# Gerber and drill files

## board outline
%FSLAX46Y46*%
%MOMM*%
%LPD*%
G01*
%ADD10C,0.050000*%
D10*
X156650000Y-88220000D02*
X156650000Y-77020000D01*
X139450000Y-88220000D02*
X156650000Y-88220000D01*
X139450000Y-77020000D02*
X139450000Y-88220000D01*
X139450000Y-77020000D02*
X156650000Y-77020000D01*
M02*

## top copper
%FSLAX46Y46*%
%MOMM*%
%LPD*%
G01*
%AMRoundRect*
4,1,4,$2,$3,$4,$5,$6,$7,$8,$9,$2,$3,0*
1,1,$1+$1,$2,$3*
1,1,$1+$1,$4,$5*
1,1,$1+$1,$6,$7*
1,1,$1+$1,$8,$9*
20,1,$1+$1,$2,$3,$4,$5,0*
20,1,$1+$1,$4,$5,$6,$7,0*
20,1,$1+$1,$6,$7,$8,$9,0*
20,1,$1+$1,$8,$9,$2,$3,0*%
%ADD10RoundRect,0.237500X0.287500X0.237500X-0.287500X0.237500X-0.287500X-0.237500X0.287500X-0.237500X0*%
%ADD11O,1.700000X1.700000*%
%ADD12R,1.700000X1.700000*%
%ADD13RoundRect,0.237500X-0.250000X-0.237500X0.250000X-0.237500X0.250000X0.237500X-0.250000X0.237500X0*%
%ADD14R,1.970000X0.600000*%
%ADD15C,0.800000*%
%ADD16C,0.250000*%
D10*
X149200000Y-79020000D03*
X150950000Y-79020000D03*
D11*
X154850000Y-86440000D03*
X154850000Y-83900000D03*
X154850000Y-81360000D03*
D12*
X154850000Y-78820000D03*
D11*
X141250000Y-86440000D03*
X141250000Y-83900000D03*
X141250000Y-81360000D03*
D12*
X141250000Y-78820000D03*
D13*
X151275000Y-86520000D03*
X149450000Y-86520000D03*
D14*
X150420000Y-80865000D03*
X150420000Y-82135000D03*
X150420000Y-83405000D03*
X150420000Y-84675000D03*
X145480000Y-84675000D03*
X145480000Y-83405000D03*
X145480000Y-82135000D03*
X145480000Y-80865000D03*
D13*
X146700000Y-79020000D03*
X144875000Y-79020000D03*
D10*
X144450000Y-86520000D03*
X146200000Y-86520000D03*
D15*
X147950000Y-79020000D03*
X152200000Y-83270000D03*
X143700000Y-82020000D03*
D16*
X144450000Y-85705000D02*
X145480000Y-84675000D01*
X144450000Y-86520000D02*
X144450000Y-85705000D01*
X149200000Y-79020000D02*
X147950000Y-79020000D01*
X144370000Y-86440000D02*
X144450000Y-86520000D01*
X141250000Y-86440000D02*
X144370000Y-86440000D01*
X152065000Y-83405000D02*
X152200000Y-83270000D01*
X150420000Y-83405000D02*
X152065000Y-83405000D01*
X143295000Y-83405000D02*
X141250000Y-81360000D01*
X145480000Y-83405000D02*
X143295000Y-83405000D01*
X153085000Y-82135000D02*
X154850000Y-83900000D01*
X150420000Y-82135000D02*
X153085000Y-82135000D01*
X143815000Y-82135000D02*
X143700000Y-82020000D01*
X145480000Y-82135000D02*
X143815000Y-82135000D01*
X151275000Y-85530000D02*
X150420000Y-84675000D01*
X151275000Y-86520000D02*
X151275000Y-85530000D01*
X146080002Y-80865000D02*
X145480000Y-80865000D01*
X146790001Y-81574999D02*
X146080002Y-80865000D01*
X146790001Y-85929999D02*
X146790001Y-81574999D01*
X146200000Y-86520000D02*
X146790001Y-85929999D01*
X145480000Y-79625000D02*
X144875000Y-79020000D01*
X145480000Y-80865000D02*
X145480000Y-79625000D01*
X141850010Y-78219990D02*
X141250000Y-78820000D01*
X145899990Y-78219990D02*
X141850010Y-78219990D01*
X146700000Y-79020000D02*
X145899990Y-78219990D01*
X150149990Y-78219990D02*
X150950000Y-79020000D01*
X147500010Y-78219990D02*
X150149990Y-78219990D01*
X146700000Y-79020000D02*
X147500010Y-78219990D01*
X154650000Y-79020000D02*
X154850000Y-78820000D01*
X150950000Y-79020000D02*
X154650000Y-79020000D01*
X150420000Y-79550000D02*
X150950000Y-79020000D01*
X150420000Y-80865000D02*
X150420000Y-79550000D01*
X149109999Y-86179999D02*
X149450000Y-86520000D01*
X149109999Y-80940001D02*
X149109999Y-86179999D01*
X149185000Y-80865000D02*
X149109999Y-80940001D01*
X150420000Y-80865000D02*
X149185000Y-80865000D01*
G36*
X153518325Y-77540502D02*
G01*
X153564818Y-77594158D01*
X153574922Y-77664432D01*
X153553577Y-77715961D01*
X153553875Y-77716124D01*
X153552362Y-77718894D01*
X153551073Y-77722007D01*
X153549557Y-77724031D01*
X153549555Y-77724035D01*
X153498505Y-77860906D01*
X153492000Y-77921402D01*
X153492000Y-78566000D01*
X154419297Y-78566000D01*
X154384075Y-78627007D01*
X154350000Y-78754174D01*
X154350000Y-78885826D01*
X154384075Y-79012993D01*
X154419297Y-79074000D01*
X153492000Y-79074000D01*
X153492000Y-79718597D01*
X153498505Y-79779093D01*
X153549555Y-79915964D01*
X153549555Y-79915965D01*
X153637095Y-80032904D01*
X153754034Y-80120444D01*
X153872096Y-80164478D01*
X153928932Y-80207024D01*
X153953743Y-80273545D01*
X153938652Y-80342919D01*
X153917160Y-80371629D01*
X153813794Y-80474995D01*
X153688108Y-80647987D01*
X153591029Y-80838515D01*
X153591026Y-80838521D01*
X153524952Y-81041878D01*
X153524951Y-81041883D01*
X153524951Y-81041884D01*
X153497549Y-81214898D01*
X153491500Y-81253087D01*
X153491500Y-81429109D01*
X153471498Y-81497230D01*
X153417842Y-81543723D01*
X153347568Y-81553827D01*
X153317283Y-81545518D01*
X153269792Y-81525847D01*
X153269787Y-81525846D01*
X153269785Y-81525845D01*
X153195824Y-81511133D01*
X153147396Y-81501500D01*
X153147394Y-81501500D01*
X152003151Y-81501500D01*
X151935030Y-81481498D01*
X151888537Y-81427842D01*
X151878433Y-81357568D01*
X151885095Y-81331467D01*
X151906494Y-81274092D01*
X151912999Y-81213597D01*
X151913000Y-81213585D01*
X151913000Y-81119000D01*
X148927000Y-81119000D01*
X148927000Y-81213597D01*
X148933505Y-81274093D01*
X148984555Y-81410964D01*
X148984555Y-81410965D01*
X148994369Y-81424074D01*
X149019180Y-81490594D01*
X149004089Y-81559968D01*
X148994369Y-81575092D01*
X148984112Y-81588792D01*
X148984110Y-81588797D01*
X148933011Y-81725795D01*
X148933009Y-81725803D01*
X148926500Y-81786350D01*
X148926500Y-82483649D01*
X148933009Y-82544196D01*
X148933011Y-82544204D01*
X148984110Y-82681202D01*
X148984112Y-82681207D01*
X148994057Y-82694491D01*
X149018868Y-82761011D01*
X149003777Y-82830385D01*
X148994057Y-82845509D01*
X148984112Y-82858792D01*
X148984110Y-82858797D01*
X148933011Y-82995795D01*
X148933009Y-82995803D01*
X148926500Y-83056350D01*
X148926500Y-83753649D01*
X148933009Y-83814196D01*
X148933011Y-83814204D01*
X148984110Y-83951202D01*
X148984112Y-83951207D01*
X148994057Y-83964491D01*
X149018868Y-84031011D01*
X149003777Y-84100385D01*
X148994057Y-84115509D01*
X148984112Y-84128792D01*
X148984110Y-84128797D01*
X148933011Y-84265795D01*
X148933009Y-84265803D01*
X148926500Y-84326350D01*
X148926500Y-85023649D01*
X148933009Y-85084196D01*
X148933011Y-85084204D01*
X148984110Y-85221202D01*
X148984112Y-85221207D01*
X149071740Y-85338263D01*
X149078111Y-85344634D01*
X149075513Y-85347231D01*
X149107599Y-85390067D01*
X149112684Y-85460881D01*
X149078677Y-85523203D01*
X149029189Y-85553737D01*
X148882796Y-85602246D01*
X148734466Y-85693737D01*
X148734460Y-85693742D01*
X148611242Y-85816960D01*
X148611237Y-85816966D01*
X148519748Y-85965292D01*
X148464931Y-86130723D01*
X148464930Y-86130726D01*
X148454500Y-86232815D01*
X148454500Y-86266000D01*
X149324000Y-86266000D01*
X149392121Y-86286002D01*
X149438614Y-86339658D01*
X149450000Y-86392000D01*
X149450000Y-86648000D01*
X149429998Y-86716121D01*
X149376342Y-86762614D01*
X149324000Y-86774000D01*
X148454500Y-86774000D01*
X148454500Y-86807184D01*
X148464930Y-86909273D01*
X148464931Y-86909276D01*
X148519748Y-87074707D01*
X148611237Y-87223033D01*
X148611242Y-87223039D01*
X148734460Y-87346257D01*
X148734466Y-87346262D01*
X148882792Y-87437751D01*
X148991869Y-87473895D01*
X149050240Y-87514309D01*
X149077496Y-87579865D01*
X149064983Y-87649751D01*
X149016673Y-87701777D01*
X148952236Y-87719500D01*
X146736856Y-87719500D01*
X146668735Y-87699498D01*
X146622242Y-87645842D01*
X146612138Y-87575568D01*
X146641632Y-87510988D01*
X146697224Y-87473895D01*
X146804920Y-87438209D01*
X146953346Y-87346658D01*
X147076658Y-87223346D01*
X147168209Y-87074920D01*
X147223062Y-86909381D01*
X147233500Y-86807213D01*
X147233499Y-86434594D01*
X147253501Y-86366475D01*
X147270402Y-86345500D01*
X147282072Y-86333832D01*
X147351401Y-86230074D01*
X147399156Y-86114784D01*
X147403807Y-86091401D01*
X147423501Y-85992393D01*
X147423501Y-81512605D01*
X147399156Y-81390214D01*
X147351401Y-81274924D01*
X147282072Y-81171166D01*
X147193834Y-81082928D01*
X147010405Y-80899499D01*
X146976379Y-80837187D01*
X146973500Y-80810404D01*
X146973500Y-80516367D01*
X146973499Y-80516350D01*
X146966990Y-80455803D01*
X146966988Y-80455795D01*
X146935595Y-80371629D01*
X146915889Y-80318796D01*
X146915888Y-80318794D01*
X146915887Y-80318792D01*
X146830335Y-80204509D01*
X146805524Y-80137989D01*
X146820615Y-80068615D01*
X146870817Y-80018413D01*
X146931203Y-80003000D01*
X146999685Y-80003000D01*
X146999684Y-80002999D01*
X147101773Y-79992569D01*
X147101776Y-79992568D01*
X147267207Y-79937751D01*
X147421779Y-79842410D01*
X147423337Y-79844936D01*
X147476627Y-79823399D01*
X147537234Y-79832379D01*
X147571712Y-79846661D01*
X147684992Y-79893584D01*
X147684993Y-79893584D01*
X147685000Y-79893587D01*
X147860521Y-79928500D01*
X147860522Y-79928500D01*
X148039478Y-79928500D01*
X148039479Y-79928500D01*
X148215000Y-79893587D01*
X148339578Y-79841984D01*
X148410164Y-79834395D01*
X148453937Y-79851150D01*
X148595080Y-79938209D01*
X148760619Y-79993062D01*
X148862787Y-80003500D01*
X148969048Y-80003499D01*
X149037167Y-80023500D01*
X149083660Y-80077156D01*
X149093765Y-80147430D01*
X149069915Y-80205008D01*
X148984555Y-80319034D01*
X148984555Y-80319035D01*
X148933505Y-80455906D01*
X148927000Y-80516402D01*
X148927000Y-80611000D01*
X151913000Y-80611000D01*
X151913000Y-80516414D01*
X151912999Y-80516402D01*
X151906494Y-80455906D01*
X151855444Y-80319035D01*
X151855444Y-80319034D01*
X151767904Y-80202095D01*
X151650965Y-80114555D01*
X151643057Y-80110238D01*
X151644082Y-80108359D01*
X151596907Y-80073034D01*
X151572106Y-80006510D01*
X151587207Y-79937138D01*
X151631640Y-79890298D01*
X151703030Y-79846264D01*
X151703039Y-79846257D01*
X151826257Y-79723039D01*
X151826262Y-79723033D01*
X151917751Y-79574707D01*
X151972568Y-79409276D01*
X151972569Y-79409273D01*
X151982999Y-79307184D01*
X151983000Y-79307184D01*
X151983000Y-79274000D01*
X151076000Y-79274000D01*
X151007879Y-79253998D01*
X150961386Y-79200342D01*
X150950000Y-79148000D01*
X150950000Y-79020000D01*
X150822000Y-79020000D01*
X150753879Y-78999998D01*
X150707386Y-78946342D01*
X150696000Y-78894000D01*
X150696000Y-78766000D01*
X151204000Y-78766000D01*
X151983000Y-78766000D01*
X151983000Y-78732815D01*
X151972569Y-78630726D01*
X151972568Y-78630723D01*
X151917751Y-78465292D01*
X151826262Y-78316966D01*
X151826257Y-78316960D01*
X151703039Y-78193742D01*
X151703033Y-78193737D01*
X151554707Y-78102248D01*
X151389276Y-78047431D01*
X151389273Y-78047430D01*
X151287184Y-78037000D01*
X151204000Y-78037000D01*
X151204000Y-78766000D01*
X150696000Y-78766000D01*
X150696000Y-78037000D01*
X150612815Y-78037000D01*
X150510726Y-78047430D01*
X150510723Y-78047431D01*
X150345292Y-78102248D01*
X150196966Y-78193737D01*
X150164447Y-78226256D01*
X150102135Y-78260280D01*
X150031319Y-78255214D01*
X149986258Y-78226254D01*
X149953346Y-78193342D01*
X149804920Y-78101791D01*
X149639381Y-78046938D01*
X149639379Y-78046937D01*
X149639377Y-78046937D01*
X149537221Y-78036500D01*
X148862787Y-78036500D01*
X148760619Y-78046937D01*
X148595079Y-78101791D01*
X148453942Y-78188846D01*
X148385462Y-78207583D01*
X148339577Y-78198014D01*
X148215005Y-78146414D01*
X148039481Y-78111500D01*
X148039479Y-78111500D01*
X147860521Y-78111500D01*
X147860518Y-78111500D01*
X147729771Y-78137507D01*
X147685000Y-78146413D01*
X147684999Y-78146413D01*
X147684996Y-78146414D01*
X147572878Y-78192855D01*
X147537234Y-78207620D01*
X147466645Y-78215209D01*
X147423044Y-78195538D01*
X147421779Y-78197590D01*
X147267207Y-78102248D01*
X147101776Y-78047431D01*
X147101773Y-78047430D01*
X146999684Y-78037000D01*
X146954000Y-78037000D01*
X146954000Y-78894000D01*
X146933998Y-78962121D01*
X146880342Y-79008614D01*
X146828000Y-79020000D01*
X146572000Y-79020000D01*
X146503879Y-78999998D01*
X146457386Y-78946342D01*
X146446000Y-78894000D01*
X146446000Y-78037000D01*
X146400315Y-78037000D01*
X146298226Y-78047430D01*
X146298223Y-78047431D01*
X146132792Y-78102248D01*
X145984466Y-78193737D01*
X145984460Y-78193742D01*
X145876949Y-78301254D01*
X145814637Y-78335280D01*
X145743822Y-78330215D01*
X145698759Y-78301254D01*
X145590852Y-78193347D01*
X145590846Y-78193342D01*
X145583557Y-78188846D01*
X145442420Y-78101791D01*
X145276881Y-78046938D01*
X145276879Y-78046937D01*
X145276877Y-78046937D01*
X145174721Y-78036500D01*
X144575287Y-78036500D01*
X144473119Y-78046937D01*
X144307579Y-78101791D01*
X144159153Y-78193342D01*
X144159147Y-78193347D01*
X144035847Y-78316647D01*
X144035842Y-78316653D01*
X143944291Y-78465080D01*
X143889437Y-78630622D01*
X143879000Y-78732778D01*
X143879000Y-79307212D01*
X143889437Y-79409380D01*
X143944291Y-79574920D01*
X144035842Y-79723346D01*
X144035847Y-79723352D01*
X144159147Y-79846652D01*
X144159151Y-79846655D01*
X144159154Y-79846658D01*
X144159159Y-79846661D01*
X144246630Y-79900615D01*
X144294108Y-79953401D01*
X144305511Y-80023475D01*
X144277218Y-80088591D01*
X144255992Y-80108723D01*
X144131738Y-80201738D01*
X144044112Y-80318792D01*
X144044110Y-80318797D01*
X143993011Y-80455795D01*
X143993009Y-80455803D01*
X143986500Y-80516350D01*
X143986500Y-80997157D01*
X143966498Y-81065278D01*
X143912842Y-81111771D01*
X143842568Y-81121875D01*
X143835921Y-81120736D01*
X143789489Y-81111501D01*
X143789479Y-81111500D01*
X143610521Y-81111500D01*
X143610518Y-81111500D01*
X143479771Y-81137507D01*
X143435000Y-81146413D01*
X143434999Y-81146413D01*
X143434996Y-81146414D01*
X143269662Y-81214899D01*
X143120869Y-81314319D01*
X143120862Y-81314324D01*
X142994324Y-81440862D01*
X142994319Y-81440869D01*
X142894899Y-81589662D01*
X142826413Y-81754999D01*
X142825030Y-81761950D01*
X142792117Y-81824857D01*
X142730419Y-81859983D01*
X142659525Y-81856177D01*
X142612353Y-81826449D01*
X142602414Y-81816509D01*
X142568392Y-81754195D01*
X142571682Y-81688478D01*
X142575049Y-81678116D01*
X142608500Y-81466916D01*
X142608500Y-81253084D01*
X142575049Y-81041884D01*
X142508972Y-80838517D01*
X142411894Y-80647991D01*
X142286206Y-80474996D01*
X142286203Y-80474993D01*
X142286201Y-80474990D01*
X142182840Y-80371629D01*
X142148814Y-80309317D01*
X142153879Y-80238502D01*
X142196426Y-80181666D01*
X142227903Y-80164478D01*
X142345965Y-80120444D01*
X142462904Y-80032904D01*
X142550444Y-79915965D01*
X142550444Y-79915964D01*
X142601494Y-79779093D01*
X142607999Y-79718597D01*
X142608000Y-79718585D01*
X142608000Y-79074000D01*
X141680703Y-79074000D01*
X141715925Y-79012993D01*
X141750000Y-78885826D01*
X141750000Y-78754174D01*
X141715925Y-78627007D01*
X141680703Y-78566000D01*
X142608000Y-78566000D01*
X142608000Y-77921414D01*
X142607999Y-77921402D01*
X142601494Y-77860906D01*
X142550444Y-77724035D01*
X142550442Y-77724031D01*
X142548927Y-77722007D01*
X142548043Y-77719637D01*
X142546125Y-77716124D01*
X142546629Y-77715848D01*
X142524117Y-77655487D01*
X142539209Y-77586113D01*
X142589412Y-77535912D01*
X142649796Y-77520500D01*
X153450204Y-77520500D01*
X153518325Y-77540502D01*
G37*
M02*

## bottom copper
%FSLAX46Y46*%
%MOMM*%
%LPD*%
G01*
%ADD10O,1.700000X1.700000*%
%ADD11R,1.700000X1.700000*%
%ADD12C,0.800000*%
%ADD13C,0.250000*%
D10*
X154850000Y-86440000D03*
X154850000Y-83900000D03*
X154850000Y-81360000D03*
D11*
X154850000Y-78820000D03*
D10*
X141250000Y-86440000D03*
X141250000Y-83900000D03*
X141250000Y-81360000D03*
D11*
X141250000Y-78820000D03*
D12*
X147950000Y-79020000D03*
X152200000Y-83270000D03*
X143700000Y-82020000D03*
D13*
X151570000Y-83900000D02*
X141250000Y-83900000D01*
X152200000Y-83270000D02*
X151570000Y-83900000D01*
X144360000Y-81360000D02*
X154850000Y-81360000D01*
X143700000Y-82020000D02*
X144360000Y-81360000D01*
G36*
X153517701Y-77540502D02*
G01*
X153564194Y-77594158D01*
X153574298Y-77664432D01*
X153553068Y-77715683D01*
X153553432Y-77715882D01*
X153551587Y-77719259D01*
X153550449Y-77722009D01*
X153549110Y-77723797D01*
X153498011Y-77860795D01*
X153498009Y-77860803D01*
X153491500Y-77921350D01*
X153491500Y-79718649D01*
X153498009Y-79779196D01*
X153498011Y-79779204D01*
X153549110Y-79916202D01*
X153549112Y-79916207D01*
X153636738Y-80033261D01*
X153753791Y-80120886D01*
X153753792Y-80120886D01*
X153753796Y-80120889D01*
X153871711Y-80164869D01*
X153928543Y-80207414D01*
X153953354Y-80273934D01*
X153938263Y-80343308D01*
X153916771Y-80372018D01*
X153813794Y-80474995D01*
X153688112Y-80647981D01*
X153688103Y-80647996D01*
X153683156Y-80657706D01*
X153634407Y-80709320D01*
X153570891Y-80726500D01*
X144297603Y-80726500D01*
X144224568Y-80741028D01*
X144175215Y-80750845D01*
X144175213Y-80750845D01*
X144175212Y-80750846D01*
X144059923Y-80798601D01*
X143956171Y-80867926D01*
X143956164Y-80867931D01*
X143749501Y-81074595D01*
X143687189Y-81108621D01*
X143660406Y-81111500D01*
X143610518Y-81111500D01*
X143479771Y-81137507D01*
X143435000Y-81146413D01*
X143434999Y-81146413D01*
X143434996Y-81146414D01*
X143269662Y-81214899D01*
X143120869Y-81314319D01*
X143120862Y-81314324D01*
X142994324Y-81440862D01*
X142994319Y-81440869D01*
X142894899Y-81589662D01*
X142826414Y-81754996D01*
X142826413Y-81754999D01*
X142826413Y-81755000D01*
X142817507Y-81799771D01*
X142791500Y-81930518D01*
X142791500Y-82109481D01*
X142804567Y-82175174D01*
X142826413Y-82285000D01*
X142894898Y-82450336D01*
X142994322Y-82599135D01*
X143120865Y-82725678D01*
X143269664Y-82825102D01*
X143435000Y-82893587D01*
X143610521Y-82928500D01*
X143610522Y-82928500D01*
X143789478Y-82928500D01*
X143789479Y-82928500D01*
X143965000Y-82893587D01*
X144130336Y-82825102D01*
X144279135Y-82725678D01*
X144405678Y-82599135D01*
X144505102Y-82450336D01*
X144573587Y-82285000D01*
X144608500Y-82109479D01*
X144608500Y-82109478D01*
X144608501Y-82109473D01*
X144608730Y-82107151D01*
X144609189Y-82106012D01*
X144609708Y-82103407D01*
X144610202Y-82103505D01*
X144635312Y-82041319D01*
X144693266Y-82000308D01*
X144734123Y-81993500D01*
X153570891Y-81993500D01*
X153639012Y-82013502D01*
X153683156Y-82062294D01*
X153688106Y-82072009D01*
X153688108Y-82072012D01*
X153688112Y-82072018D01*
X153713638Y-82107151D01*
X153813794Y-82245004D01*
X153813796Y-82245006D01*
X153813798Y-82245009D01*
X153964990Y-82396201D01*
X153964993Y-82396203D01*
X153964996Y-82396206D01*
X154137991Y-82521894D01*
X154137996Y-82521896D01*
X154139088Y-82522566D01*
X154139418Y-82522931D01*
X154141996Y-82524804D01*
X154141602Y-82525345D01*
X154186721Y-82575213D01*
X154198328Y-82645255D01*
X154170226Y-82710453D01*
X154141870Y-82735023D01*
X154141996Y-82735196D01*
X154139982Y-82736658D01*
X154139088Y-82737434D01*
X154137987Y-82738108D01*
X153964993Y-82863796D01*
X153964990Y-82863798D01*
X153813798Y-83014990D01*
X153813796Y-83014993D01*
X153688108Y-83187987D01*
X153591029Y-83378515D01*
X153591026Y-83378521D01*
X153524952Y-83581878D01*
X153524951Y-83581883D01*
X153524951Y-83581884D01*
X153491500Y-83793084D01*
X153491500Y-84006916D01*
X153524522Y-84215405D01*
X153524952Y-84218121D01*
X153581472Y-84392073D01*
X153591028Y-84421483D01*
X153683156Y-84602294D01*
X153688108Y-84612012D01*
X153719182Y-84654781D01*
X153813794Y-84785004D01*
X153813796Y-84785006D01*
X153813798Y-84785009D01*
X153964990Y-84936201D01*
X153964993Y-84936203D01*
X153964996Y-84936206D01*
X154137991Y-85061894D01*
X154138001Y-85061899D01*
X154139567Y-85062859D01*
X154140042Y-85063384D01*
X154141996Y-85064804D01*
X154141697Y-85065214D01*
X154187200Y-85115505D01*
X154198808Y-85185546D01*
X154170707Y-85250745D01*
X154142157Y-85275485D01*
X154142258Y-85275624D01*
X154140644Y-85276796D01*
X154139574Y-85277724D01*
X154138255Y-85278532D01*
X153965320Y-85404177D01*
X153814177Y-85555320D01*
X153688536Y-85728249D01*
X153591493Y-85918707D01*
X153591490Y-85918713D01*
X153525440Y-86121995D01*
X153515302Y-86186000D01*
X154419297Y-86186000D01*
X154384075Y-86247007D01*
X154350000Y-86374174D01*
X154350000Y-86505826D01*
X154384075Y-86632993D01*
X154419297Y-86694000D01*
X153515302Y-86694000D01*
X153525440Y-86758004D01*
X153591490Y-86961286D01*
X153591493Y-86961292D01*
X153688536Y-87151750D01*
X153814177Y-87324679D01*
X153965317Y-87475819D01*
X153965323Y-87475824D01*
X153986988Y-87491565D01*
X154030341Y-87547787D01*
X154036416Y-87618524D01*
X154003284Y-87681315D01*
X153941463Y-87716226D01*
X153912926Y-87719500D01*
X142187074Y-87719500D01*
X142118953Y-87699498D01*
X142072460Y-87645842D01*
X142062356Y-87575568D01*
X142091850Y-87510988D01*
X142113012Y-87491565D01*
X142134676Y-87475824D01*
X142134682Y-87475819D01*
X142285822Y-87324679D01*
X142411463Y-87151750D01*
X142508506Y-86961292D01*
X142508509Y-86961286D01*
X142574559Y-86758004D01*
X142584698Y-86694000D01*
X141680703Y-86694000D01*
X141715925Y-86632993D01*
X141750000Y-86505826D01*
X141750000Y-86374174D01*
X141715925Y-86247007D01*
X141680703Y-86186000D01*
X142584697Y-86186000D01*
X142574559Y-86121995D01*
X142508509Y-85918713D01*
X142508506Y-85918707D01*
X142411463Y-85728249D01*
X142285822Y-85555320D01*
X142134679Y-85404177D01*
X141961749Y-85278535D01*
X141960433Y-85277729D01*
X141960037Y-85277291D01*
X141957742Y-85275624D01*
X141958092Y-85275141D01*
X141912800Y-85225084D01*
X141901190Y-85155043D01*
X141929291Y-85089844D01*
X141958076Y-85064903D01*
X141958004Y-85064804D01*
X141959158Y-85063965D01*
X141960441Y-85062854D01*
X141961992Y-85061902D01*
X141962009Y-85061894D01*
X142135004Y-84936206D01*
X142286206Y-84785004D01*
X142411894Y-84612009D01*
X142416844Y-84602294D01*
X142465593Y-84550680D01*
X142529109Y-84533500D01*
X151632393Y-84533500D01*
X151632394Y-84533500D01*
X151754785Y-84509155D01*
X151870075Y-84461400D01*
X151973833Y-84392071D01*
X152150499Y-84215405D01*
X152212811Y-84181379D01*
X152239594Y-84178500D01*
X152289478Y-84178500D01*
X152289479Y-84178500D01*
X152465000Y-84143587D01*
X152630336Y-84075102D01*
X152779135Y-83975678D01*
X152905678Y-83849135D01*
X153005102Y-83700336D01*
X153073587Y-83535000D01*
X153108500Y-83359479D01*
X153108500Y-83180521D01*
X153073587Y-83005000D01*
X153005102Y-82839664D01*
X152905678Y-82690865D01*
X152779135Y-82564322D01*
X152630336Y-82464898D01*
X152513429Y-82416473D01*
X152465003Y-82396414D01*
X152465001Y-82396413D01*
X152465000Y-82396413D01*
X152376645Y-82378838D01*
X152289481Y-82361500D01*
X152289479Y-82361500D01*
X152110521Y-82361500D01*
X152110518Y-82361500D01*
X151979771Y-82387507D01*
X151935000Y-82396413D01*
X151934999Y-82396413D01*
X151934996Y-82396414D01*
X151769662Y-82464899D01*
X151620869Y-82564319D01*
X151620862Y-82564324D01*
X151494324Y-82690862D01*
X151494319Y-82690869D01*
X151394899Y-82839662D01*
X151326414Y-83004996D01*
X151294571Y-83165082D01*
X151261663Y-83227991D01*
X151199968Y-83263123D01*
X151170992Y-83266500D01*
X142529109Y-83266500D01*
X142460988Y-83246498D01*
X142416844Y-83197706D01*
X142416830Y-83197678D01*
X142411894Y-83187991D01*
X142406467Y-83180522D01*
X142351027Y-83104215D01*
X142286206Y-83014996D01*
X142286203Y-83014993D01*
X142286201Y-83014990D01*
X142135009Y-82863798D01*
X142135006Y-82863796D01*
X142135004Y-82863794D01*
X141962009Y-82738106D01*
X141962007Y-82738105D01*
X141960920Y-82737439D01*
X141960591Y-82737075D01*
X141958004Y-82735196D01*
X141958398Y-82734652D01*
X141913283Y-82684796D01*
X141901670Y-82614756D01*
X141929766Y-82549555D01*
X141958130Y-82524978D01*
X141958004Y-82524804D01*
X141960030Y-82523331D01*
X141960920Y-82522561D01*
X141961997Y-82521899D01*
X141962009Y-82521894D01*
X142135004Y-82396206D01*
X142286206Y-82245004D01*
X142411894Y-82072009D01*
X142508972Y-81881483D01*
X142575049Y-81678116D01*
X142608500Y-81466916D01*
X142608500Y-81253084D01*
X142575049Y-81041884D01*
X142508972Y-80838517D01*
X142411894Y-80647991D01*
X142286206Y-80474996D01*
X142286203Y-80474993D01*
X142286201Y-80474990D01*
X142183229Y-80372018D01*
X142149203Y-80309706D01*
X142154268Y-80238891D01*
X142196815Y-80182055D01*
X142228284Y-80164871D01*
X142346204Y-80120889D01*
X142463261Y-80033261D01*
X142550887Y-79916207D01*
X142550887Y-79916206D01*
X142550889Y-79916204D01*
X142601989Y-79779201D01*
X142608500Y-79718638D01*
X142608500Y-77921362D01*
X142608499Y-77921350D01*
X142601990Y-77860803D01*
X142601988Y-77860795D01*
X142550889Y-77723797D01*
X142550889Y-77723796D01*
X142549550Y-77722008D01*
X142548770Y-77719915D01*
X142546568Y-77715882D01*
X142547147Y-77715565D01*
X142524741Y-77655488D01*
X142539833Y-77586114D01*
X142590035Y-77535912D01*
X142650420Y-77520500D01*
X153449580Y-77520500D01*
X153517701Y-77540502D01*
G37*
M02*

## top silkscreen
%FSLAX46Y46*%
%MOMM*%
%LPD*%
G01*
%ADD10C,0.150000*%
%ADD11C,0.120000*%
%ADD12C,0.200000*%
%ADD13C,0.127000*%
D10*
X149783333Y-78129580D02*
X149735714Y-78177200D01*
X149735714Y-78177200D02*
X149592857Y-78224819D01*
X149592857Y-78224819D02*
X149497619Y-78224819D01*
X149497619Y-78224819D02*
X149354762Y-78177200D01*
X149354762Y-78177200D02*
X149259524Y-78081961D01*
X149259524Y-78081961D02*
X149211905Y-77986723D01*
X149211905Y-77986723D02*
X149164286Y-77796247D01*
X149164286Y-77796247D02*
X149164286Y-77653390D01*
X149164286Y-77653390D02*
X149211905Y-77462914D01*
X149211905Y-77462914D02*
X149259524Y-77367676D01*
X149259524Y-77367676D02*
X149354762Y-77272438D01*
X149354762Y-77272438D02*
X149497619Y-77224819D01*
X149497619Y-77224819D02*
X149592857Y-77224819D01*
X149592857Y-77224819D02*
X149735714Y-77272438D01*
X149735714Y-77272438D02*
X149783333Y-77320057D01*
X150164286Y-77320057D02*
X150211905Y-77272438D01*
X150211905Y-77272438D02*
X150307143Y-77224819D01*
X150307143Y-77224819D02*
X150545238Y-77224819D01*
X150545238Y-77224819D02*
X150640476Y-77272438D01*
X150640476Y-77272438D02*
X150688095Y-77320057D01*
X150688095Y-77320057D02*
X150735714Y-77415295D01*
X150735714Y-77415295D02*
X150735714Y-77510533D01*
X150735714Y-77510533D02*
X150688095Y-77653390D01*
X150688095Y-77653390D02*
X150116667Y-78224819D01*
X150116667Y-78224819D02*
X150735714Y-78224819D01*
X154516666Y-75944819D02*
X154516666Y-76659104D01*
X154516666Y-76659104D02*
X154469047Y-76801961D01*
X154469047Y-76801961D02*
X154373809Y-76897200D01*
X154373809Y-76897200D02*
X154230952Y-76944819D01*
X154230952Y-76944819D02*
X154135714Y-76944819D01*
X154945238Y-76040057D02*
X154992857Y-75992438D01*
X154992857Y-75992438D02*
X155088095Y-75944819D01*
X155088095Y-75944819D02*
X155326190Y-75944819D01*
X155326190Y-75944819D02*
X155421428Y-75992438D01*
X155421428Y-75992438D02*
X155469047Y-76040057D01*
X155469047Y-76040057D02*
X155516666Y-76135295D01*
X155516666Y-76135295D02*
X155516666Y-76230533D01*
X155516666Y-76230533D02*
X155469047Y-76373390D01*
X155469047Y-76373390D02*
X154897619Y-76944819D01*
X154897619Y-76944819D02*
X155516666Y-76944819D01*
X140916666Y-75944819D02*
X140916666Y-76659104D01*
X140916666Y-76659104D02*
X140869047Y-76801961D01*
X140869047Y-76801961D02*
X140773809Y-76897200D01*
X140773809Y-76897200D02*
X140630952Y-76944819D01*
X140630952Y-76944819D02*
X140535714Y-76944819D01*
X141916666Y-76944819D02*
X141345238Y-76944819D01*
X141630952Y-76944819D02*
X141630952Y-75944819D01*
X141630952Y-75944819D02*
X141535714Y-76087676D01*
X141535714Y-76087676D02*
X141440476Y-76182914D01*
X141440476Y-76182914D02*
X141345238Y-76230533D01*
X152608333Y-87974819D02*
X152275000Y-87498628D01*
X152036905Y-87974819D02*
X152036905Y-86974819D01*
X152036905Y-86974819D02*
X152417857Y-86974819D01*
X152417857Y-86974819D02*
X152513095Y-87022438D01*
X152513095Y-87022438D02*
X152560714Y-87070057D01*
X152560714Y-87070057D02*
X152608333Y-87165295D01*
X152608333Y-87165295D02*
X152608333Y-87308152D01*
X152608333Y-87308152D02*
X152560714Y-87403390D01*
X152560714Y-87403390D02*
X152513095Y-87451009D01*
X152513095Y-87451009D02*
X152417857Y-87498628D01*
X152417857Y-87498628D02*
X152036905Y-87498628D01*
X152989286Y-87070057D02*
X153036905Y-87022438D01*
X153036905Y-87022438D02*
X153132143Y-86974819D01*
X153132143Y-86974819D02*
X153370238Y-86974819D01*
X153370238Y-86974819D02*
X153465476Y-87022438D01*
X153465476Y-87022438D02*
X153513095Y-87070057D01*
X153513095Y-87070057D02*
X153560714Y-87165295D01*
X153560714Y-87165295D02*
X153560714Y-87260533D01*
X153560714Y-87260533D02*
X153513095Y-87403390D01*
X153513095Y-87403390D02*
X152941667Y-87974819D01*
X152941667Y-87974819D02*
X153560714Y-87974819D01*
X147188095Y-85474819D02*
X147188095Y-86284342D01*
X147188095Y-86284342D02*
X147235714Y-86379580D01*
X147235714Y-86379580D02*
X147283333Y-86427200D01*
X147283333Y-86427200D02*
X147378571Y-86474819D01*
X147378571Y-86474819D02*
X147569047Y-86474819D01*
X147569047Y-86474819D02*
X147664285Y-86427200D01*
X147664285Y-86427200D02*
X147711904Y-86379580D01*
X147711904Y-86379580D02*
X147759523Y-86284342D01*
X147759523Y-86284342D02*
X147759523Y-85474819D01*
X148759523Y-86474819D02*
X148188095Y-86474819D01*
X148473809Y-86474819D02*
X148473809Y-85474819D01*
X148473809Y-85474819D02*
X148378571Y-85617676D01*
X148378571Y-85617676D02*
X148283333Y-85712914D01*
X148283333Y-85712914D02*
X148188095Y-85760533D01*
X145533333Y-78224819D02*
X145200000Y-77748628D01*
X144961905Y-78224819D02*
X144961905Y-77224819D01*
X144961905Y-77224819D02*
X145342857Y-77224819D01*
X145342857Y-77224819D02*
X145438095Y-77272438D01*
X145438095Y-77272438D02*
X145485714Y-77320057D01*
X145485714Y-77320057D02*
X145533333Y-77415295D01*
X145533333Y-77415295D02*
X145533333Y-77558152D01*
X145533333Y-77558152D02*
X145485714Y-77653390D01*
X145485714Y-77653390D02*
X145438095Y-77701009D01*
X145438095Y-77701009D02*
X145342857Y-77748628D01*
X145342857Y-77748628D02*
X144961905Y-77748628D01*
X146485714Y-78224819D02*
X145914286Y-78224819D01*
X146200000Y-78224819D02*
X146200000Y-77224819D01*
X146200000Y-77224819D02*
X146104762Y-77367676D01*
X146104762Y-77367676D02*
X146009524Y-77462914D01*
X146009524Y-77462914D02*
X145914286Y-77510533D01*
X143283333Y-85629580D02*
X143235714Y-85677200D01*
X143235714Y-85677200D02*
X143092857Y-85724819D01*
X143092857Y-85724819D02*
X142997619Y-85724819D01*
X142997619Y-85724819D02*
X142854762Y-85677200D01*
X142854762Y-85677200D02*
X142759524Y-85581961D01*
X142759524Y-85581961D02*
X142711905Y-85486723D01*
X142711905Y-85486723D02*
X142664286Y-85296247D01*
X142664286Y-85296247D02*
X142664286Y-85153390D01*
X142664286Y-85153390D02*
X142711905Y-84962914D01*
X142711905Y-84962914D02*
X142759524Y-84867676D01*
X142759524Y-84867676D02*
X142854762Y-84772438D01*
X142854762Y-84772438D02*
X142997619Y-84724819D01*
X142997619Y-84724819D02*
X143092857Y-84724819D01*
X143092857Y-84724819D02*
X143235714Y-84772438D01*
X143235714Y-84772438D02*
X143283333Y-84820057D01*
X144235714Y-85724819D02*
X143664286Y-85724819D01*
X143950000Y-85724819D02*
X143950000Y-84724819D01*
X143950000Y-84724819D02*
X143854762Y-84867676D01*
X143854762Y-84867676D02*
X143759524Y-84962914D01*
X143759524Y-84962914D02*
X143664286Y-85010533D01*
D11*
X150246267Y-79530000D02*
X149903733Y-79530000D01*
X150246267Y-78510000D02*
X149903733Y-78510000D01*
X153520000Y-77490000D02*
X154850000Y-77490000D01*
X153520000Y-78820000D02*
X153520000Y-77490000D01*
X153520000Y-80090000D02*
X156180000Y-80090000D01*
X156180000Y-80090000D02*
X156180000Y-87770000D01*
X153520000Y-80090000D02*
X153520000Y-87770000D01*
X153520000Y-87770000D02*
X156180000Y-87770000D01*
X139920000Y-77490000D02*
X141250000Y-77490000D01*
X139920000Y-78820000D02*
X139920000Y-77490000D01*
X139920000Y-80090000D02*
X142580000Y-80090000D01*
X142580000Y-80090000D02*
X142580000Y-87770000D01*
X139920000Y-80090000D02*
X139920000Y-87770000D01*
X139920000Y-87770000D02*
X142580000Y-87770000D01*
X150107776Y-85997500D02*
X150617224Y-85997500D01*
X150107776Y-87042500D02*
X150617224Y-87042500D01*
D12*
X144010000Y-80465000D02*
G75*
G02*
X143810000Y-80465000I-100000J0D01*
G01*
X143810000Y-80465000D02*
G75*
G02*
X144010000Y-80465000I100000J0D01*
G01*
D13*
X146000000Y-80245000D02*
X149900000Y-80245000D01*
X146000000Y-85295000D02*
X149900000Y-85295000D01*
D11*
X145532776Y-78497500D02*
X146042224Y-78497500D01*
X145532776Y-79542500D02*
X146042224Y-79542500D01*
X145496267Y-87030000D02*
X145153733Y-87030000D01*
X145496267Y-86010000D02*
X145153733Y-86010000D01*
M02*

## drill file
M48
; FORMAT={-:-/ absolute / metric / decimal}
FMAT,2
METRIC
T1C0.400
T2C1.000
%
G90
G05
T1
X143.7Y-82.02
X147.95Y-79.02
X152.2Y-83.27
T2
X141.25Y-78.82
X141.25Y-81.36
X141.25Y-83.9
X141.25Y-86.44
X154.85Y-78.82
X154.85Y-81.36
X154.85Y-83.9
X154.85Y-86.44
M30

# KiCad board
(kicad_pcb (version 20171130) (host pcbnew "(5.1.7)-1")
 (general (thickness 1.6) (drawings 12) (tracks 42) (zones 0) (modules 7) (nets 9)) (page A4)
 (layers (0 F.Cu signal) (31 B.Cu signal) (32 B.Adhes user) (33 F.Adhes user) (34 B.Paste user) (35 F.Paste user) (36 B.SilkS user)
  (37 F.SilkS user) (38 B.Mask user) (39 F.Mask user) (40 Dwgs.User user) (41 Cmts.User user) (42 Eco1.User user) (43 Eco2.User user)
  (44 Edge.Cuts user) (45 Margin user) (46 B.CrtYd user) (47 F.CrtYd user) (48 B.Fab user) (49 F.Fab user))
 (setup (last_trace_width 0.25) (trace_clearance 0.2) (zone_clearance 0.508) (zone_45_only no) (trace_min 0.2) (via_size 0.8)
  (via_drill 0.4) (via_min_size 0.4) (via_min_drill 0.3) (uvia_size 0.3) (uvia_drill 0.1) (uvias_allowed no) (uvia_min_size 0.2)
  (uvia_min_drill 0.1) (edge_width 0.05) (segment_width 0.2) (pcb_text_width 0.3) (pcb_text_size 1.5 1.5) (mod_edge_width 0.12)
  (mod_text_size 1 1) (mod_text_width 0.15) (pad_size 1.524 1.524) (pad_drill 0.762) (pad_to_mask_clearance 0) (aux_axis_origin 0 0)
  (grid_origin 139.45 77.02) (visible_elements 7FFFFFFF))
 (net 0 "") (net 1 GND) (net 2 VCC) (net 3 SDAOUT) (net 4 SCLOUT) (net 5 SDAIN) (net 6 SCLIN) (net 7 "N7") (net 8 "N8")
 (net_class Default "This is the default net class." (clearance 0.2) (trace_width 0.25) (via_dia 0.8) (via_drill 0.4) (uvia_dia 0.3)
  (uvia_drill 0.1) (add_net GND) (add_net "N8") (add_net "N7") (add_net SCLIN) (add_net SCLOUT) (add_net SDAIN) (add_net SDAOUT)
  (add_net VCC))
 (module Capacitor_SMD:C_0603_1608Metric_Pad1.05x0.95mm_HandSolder (layer F.Cu) (at 150.075 79.02 180)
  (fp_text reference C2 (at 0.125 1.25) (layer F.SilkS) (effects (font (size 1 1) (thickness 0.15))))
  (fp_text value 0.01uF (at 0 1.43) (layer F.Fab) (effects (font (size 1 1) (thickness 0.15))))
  (fp_line (start -0.171267 -0.51) (end 0.171267 -0.51) (layer F.SilkS) (width 0.12))
  (fp_line (start -0.171267 0.51) (end 0.171267 0.51) (layer F.SilkS) (width 0.12))
  (pad 2 smd roundrect (at 0.875 0 180) (size 1.05 0.95) (layers F.Cu F.Paste F.Mask) (roundrect_rratio 0.25) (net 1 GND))
  (pad 1 smd roundrect (at -0.875 0 180) (size 1.05 0.95) (layers F.Cu F.Paste F.Mask) (roundrect_rratio 0.25) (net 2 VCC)))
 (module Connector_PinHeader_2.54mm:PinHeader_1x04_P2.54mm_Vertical (layer F.Cu) (at 154.85 78.82)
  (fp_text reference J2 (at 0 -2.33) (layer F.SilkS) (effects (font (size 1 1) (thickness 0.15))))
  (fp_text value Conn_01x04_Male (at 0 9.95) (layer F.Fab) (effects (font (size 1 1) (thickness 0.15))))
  (fp_line (start -1.33 -1.33) (end 0 -1.33) (layer F.SilkS) (width 0.12))
  (fp_line (start -1.33 0) (end -1.33 -1.33) (layer F.SilkS) (width 0.12))
  (fp_line (start -1.33 1.27) (end 1.33 1.27) (layer F.SilkS) (width 0.12))
  (fp_line (start 1.33 1.27) (end 1.33 8.95) (layer F.SilkS) (width 0.12))
  (fp_line (start -1.33 1.27) (end -1.33 8.95) (layer F.SilkS) (width 0.12))
  (fp_line (start -1.33 8.95) (end 1.33 8.95) (layer F.SilkS) (width 0.12))
  (pad 4 thru_hole oval (at 0 7.62) (size 1.7 1.7) (drill 1) (layers *.Cu *.Mask) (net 1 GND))
  (pad 3 thru_hole oval (at 0 5.08) (size 1.7 1.7) (drill 1) (layers *.Cu *.Mask) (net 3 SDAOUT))
  (pad 2 thru_hole oval (at 0 2.54) (size 1.7 1.7) (drill 1) (layers *.Cu *.Mask) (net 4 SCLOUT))
  (pad 1 thru_hole rect (at 0 0) (size 1.7 1.7) (drill 1) (layers *.Cu *.Mask) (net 2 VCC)))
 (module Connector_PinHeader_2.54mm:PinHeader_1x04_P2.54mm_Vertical (layer F.Cu) (at 141.25 78.82)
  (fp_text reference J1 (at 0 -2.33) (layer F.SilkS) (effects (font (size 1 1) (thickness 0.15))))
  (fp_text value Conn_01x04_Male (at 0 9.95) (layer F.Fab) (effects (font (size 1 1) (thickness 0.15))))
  (fp_line (start -1.33 -1.33) (end 0 -1.33) (layer F.SilkS) (width 0.12))
  (fp_line (start -1.33 0) (end -1.33 -1.33) (layer F.SilkS) (width 0.12))
  (fp_line (start -1.33 1.27) (end 1.33 1.27) (layer F.SilkS) (width 0.12))
  (fp_line (start 1.33 1.27) (end 1.33 8.95) (layer F.SilkS) (width 0.12))
  (fp_line (start -1.33 1.27) (end -1.33 8.95) (layer F.SilkS) (width 0.12))
  (fp_line (start -1.33 8.95) (end 1.33 8.95) (layer F.SilkS) (width 0.12))
  (pad 4 thru_hole oval (at 0 7.62) (size 1.7 1.7) (drill 1) (layers *.Cu *.Mask) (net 1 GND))
  (pad 3 thru_hole oval (at 0 5.08) (size 1.7 1.7) (drill 1) (layers *.Cu *.Mask) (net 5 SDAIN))
  (pad 2 thru_hole oval (at 0 2.54) (size 1.7 1.7) (drill 1) (layers *.Cu *.Mask) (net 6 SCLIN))
  (pad 1 thru_hole rect (at 0 0) (size 1.7 1.7) (drill 1) (layers *.Cu *.Mask) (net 2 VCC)))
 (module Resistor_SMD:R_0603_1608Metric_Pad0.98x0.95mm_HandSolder (layer F.Cu) (at 150.3625 86.52)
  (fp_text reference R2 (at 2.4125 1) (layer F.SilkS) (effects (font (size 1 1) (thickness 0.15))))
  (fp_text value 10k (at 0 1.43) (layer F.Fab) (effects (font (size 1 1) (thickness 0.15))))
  (fp_line (start -0.254724 -0.5225) (end 0.254724 -0.5225) (layer F.SilkS) (width 0.12))
  (fp_line (start -0.254724 0.5225) (end 0.254724 0.5225) (layer F.SilkS) (width 0.12))
  (pad 2 smd roundrect (at 0.9125 0) (size 0.975 0.95) (layers F.Cu F.Paste F.Mask) (roundrect_rratio 0.25) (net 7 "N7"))
  (pad 1 smd roundrect (at -0.9125 0) (size 0.975 0.95) (layers F.Cu F.Paste F.Mask) (roundrect_rratio 0.25) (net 2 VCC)))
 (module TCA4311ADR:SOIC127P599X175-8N (layer F.Cu) (at 147.95 82.77)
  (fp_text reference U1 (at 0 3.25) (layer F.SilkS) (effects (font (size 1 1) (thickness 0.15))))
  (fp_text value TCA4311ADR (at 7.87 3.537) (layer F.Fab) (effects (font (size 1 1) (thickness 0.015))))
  (fp_circle (center -4.04 -2.305) (end -3.94 -2.305) (layer F.SilkS) (width 0.2))
  (fp_line (start -1.95 -2.525) (end 1.95 -2.525) (layer F.SilkS) (width 0.127))
  (fp_line (start -1.95 2.525) (end 1.95 2.525) (layer F.SilkS) (width 0.127))
  (pad 8 smd rect (at 2.47 -1.905) (size 1.97 0.6) (layers F.Cu F.Paste F.Mask) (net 2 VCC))
  (pad 7 smd rect (at 2.47 -0.635) (size 1.97 0.6) (layers F.Cu F.Paste F.Mask) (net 3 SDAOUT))
  (pad 6 smd rect (at 2.47 0.635) (size 1.97 0.6) (layers F.Cu F.Paste F.Mask) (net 5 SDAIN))
  (pad 5 smd rect (at 2.47 1.905) (size 1.97 0.6) (layers F.Cu F.Paste F.Mask) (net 7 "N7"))
  (pad 4 smd rect (at -2.47 1.905) (size 1.97 0.6) (layers F.Cu F.Paste F.Mask) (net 1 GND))
  (pad 3 smd rect (at -2.47 0.635) (size 1.97 0.6) (layers F.Cu F.Paste F.Mask) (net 6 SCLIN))
  (pad 2 smd rect (at -2.47 -0.635) (size 1.97 0.6) (layers F.Cu F.Paste F.Mask) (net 4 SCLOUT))
  (pad 1 smd rect (at -2.47 -1.905) (size 1.97 0.6) (layers F.Cu F.Paste F.Mask) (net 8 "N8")))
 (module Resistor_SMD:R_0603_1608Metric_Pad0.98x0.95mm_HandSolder (layer F.Cu) (at 145.7875 79.02)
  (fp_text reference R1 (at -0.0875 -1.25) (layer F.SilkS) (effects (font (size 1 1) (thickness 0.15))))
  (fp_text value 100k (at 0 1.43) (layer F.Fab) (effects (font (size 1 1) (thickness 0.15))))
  (fp_line (start -0.254724 -0.5225) (end 0.254724 -0.5225) (layer F.SilkS) (width 0.12))
  (fp_line (start -0.254724 0.5225) (end 0.254724 0.5225) (layer F.SilkS) (width 0.12))
  (pad 2 smd roundrect (at 0.9125 0) (size 0.975 0.95) (layers F.Cu F.Paste F.Mask) (roundrect_rratio 0.25) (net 2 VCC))
  (pad 1 smd roundrect (at -0.9125 0) (size 0.975 0.95) (layers F.Cu F.Paste F.Mask) (roundrect_rratio 0.25) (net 8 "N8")))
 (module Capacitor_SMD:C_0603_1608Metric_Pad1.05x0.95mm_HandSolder (layer F.Cu) (at 145.325 86.52 180)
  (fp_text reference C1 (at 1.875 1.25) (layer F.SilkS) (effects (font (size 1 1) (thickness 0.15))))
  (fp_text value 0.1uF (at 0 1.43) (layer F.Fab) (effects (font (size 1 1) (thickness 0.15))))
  (fp_line (start -0.171267 -0.51) (end 0.171267 -0.51) (layer F.SilkS) (width 0.12))
  (fp_line (start -0.171267 0.51) (end 0.171267 0.51) (layer F.SilkS) (width 0.12))
  (pad 2 smd roundrect (at 0.875 0 180) (size 1.05 0.95) (layers F.Cu F.Paste F.Mask) (roundrect_rratio 0.25) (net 1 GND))
  (pad 1 smd roundrect (at -0.875 0 180) (size 1.05 0.95) (layers F.Cu F.Paste F.Mask) (roundrect_rratio 0.25) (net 8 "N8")))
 (gr_line (start 156.65 88.22) (end 156.65 77.02) (layer Edge.Cuts) (width 0.05))
 (gr_line (start 139.45 88.22) (end 156.65 88.22) (layer Edge.Cuts) (width 0.05))
 (gr_line (start 139.45 77.02) (end 139.45 88.22) (layer Edge.Cuts) (width 0.05))
 (gr_line (start 139.45 77.02) (end 156.65 77.02) (layer Edge.Cuts) (width 0.05))
 (segment (start 144.45 85.705) (end 145.48 84.675) (width 0.25) (layer F.Cu) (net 1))
 (segment (start 144.45 86.52) (end 144.45 85.705) (width 0.25) (layer F.Cu) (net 1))
 (via (at 147.95 79.02) (size 0.8) (drill 0.4) (layers F.Cu B.Cu) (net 1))
 (segment (start 149.2 79.02) (end 147.95 79.02) (width 0.25) (layer F.Cu) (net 1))
 (segment (start 144.37 86.44) (end 144.45 86.52) (width 0.25) (layer F.Cu) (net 1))
 (segment (start 141.25 86.44) (end 144.37 86.44) (width 0.25) (layer F.Cu) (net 1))
 (via (at 152.2 83.27) (size 0.8) (drill 0.4) (layers F.Cu B.Cu) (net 5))
 (segment (start 152.065 83.405) (end 152.2 83.27) (width 0.25) (layer F.Cu) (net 5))
 (segment (start 150.42 83.405) (end 152.065 83.405) (width 0.25) (layer F.Cu) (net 5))
 (segment (start 151.57 83.9) (end 141.25 83.9) (width 0.25) (layer B.Cu) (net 5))
 (segment (start 152.2 83.27) (end 151.57 83.9) (width 0.25) (layer B.Cu) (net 5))
 (segment (start 143.295 83.405) (end 141.25 81.36) (width 0.25) (layer F.Cu) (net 6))
 (segment (start 145.48 83.405) (end 143.295 83.405) (width 0.25) (layer F.Cu) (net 6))
 (segment (start 153.085 82.135) (end 154.85 83.9) (width 0.25) (layer F.Cu) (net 3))
 (segment (start 150.42 82.135) (end 153.085 82.135) (width 0.25) (layer F.Cu) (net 3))
 (via (at 143.7 82.02) (size 0.8) (drill 0.4) (layers F.Cu B.Cu) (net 4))
 (segment (start 143.815 82.135) (end 143.7 82.02) (width 0.25) (layer F.Cu) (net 4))
 (segment (start 145.48 82.135) (end 143.815 82.135) (width 0.25) (layer F.Cu) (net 4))
 (segment (start 144.36 81.36) (end 154.85 81.36) (width 0.25) (layer B.Cu) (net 4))
 (segment (start 143.7 82.02) (end 144.36 81.36) (width 0.25) (layer B.Cu) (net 4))
 (segment (start 151.275 85.53) (end 150.42 84.675) (width 0.25) (layer F.Cu) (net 7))
 (segment (start 151.275 86.52) (end 151.275 85.53) (width 0.25) (layer F.Cu) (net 7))
 (segment (start 146.080002 80.865) (end 145.48 80.865) (width 0.25) (layer F.Cu) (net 8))
 (segment (start 146.790001 81.574999) (end 146.080002 80.865) (width 0.25) (layer F.Cu) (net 8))
 (segment (start 146.790001 85.929999) (end 146.790001 81.574999) (width 0.25) (layer F.Cu) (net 8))
 (segment (start 146.2 86.52) (end 146.790001 85.929999) (width 0.25) (layer F.Cu) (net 8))
 (segment (start 145.48 79.625) (end 144.875 79.02) (width 0.25) (layer F.Cu) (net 8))
 (segment (start 145.48 80.865) (end 145.48 79.625) (width 0.25) (layer F.Cu) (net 8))
 (segment (start 141.85001 78.21999) (end 141.25 78.82) (width 0.25) (layer F.Cu) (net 2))
 (segment (start 145.89999 78.21999) (end 141.85001 78.21999) (width 0.25) (layer F.Cu) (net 2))
 (segment (start 146.7 79.02) (end 145.89999 78.21999) (width 0.25) (layer F.Cu) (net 2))
 (segment (start 150.14999 78.21999) (end 150.95 79.02) (width 0.25) (layer F.Cu) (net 2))
 (segment (start 147.50001 78.21999) (end 150.14999 78.21999) (width 0.25) (layer F.Cu) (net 2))
 (segment (start 146.7 79.02) (end 147.50001 78.21999) (width 0.25) (layer F.Cu) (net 2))
 (segment (start 154.65 79.02) (end 154.85 78.82) (width 0.25) (layer F.Cu) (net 2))
 (segment (start 150.95 79.02) (end 154.65 79.02) (width 0.25) (layer F.Cu) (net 2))
 (segment (start 150.42 79.55) (end 150.95 79.02) (width 0.25) (layer F.Cu) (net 2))
 (segment (start 150.42 80.865) (end 150.42 79.55) (width 0.25) (layer F.Cu) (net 2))
 (segment (start 149.109999 86.179999) (end 149.45 86.52) (width 0.25) (layer F.Cu) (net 2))
 (segment (start 149.109999 80.940001) (end 149.109999 86.179999) (width 0.25) (layer F.Cu) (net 2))
 (segment (start 149.185 80.865) (end 149.109999 80.940001) (width 0.25) (layer F.Cu) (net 2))
 (segment (start 150.42 80.865) (end 149.185 80.865) (width 0.25) (layer F.Cu) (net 2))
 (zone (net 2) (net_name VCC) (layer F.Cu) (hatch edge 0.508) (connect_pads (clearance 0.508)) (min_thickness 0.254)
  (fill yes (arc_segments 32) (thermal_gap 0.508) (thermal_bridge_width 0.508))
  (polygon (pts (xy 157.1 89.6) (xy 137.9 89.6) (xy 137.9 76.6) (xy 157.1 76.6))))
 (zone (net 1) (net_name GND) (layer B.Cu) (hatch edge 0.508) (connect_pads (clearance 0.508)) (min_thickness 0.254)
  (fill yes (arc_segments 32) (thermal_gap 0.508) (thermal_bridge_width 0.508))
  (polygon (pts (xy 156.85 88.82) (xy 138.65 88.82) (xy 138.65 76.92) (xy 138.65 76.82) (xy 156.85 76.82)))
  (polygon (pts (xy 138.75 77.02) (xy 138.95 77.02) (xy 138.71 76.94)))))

